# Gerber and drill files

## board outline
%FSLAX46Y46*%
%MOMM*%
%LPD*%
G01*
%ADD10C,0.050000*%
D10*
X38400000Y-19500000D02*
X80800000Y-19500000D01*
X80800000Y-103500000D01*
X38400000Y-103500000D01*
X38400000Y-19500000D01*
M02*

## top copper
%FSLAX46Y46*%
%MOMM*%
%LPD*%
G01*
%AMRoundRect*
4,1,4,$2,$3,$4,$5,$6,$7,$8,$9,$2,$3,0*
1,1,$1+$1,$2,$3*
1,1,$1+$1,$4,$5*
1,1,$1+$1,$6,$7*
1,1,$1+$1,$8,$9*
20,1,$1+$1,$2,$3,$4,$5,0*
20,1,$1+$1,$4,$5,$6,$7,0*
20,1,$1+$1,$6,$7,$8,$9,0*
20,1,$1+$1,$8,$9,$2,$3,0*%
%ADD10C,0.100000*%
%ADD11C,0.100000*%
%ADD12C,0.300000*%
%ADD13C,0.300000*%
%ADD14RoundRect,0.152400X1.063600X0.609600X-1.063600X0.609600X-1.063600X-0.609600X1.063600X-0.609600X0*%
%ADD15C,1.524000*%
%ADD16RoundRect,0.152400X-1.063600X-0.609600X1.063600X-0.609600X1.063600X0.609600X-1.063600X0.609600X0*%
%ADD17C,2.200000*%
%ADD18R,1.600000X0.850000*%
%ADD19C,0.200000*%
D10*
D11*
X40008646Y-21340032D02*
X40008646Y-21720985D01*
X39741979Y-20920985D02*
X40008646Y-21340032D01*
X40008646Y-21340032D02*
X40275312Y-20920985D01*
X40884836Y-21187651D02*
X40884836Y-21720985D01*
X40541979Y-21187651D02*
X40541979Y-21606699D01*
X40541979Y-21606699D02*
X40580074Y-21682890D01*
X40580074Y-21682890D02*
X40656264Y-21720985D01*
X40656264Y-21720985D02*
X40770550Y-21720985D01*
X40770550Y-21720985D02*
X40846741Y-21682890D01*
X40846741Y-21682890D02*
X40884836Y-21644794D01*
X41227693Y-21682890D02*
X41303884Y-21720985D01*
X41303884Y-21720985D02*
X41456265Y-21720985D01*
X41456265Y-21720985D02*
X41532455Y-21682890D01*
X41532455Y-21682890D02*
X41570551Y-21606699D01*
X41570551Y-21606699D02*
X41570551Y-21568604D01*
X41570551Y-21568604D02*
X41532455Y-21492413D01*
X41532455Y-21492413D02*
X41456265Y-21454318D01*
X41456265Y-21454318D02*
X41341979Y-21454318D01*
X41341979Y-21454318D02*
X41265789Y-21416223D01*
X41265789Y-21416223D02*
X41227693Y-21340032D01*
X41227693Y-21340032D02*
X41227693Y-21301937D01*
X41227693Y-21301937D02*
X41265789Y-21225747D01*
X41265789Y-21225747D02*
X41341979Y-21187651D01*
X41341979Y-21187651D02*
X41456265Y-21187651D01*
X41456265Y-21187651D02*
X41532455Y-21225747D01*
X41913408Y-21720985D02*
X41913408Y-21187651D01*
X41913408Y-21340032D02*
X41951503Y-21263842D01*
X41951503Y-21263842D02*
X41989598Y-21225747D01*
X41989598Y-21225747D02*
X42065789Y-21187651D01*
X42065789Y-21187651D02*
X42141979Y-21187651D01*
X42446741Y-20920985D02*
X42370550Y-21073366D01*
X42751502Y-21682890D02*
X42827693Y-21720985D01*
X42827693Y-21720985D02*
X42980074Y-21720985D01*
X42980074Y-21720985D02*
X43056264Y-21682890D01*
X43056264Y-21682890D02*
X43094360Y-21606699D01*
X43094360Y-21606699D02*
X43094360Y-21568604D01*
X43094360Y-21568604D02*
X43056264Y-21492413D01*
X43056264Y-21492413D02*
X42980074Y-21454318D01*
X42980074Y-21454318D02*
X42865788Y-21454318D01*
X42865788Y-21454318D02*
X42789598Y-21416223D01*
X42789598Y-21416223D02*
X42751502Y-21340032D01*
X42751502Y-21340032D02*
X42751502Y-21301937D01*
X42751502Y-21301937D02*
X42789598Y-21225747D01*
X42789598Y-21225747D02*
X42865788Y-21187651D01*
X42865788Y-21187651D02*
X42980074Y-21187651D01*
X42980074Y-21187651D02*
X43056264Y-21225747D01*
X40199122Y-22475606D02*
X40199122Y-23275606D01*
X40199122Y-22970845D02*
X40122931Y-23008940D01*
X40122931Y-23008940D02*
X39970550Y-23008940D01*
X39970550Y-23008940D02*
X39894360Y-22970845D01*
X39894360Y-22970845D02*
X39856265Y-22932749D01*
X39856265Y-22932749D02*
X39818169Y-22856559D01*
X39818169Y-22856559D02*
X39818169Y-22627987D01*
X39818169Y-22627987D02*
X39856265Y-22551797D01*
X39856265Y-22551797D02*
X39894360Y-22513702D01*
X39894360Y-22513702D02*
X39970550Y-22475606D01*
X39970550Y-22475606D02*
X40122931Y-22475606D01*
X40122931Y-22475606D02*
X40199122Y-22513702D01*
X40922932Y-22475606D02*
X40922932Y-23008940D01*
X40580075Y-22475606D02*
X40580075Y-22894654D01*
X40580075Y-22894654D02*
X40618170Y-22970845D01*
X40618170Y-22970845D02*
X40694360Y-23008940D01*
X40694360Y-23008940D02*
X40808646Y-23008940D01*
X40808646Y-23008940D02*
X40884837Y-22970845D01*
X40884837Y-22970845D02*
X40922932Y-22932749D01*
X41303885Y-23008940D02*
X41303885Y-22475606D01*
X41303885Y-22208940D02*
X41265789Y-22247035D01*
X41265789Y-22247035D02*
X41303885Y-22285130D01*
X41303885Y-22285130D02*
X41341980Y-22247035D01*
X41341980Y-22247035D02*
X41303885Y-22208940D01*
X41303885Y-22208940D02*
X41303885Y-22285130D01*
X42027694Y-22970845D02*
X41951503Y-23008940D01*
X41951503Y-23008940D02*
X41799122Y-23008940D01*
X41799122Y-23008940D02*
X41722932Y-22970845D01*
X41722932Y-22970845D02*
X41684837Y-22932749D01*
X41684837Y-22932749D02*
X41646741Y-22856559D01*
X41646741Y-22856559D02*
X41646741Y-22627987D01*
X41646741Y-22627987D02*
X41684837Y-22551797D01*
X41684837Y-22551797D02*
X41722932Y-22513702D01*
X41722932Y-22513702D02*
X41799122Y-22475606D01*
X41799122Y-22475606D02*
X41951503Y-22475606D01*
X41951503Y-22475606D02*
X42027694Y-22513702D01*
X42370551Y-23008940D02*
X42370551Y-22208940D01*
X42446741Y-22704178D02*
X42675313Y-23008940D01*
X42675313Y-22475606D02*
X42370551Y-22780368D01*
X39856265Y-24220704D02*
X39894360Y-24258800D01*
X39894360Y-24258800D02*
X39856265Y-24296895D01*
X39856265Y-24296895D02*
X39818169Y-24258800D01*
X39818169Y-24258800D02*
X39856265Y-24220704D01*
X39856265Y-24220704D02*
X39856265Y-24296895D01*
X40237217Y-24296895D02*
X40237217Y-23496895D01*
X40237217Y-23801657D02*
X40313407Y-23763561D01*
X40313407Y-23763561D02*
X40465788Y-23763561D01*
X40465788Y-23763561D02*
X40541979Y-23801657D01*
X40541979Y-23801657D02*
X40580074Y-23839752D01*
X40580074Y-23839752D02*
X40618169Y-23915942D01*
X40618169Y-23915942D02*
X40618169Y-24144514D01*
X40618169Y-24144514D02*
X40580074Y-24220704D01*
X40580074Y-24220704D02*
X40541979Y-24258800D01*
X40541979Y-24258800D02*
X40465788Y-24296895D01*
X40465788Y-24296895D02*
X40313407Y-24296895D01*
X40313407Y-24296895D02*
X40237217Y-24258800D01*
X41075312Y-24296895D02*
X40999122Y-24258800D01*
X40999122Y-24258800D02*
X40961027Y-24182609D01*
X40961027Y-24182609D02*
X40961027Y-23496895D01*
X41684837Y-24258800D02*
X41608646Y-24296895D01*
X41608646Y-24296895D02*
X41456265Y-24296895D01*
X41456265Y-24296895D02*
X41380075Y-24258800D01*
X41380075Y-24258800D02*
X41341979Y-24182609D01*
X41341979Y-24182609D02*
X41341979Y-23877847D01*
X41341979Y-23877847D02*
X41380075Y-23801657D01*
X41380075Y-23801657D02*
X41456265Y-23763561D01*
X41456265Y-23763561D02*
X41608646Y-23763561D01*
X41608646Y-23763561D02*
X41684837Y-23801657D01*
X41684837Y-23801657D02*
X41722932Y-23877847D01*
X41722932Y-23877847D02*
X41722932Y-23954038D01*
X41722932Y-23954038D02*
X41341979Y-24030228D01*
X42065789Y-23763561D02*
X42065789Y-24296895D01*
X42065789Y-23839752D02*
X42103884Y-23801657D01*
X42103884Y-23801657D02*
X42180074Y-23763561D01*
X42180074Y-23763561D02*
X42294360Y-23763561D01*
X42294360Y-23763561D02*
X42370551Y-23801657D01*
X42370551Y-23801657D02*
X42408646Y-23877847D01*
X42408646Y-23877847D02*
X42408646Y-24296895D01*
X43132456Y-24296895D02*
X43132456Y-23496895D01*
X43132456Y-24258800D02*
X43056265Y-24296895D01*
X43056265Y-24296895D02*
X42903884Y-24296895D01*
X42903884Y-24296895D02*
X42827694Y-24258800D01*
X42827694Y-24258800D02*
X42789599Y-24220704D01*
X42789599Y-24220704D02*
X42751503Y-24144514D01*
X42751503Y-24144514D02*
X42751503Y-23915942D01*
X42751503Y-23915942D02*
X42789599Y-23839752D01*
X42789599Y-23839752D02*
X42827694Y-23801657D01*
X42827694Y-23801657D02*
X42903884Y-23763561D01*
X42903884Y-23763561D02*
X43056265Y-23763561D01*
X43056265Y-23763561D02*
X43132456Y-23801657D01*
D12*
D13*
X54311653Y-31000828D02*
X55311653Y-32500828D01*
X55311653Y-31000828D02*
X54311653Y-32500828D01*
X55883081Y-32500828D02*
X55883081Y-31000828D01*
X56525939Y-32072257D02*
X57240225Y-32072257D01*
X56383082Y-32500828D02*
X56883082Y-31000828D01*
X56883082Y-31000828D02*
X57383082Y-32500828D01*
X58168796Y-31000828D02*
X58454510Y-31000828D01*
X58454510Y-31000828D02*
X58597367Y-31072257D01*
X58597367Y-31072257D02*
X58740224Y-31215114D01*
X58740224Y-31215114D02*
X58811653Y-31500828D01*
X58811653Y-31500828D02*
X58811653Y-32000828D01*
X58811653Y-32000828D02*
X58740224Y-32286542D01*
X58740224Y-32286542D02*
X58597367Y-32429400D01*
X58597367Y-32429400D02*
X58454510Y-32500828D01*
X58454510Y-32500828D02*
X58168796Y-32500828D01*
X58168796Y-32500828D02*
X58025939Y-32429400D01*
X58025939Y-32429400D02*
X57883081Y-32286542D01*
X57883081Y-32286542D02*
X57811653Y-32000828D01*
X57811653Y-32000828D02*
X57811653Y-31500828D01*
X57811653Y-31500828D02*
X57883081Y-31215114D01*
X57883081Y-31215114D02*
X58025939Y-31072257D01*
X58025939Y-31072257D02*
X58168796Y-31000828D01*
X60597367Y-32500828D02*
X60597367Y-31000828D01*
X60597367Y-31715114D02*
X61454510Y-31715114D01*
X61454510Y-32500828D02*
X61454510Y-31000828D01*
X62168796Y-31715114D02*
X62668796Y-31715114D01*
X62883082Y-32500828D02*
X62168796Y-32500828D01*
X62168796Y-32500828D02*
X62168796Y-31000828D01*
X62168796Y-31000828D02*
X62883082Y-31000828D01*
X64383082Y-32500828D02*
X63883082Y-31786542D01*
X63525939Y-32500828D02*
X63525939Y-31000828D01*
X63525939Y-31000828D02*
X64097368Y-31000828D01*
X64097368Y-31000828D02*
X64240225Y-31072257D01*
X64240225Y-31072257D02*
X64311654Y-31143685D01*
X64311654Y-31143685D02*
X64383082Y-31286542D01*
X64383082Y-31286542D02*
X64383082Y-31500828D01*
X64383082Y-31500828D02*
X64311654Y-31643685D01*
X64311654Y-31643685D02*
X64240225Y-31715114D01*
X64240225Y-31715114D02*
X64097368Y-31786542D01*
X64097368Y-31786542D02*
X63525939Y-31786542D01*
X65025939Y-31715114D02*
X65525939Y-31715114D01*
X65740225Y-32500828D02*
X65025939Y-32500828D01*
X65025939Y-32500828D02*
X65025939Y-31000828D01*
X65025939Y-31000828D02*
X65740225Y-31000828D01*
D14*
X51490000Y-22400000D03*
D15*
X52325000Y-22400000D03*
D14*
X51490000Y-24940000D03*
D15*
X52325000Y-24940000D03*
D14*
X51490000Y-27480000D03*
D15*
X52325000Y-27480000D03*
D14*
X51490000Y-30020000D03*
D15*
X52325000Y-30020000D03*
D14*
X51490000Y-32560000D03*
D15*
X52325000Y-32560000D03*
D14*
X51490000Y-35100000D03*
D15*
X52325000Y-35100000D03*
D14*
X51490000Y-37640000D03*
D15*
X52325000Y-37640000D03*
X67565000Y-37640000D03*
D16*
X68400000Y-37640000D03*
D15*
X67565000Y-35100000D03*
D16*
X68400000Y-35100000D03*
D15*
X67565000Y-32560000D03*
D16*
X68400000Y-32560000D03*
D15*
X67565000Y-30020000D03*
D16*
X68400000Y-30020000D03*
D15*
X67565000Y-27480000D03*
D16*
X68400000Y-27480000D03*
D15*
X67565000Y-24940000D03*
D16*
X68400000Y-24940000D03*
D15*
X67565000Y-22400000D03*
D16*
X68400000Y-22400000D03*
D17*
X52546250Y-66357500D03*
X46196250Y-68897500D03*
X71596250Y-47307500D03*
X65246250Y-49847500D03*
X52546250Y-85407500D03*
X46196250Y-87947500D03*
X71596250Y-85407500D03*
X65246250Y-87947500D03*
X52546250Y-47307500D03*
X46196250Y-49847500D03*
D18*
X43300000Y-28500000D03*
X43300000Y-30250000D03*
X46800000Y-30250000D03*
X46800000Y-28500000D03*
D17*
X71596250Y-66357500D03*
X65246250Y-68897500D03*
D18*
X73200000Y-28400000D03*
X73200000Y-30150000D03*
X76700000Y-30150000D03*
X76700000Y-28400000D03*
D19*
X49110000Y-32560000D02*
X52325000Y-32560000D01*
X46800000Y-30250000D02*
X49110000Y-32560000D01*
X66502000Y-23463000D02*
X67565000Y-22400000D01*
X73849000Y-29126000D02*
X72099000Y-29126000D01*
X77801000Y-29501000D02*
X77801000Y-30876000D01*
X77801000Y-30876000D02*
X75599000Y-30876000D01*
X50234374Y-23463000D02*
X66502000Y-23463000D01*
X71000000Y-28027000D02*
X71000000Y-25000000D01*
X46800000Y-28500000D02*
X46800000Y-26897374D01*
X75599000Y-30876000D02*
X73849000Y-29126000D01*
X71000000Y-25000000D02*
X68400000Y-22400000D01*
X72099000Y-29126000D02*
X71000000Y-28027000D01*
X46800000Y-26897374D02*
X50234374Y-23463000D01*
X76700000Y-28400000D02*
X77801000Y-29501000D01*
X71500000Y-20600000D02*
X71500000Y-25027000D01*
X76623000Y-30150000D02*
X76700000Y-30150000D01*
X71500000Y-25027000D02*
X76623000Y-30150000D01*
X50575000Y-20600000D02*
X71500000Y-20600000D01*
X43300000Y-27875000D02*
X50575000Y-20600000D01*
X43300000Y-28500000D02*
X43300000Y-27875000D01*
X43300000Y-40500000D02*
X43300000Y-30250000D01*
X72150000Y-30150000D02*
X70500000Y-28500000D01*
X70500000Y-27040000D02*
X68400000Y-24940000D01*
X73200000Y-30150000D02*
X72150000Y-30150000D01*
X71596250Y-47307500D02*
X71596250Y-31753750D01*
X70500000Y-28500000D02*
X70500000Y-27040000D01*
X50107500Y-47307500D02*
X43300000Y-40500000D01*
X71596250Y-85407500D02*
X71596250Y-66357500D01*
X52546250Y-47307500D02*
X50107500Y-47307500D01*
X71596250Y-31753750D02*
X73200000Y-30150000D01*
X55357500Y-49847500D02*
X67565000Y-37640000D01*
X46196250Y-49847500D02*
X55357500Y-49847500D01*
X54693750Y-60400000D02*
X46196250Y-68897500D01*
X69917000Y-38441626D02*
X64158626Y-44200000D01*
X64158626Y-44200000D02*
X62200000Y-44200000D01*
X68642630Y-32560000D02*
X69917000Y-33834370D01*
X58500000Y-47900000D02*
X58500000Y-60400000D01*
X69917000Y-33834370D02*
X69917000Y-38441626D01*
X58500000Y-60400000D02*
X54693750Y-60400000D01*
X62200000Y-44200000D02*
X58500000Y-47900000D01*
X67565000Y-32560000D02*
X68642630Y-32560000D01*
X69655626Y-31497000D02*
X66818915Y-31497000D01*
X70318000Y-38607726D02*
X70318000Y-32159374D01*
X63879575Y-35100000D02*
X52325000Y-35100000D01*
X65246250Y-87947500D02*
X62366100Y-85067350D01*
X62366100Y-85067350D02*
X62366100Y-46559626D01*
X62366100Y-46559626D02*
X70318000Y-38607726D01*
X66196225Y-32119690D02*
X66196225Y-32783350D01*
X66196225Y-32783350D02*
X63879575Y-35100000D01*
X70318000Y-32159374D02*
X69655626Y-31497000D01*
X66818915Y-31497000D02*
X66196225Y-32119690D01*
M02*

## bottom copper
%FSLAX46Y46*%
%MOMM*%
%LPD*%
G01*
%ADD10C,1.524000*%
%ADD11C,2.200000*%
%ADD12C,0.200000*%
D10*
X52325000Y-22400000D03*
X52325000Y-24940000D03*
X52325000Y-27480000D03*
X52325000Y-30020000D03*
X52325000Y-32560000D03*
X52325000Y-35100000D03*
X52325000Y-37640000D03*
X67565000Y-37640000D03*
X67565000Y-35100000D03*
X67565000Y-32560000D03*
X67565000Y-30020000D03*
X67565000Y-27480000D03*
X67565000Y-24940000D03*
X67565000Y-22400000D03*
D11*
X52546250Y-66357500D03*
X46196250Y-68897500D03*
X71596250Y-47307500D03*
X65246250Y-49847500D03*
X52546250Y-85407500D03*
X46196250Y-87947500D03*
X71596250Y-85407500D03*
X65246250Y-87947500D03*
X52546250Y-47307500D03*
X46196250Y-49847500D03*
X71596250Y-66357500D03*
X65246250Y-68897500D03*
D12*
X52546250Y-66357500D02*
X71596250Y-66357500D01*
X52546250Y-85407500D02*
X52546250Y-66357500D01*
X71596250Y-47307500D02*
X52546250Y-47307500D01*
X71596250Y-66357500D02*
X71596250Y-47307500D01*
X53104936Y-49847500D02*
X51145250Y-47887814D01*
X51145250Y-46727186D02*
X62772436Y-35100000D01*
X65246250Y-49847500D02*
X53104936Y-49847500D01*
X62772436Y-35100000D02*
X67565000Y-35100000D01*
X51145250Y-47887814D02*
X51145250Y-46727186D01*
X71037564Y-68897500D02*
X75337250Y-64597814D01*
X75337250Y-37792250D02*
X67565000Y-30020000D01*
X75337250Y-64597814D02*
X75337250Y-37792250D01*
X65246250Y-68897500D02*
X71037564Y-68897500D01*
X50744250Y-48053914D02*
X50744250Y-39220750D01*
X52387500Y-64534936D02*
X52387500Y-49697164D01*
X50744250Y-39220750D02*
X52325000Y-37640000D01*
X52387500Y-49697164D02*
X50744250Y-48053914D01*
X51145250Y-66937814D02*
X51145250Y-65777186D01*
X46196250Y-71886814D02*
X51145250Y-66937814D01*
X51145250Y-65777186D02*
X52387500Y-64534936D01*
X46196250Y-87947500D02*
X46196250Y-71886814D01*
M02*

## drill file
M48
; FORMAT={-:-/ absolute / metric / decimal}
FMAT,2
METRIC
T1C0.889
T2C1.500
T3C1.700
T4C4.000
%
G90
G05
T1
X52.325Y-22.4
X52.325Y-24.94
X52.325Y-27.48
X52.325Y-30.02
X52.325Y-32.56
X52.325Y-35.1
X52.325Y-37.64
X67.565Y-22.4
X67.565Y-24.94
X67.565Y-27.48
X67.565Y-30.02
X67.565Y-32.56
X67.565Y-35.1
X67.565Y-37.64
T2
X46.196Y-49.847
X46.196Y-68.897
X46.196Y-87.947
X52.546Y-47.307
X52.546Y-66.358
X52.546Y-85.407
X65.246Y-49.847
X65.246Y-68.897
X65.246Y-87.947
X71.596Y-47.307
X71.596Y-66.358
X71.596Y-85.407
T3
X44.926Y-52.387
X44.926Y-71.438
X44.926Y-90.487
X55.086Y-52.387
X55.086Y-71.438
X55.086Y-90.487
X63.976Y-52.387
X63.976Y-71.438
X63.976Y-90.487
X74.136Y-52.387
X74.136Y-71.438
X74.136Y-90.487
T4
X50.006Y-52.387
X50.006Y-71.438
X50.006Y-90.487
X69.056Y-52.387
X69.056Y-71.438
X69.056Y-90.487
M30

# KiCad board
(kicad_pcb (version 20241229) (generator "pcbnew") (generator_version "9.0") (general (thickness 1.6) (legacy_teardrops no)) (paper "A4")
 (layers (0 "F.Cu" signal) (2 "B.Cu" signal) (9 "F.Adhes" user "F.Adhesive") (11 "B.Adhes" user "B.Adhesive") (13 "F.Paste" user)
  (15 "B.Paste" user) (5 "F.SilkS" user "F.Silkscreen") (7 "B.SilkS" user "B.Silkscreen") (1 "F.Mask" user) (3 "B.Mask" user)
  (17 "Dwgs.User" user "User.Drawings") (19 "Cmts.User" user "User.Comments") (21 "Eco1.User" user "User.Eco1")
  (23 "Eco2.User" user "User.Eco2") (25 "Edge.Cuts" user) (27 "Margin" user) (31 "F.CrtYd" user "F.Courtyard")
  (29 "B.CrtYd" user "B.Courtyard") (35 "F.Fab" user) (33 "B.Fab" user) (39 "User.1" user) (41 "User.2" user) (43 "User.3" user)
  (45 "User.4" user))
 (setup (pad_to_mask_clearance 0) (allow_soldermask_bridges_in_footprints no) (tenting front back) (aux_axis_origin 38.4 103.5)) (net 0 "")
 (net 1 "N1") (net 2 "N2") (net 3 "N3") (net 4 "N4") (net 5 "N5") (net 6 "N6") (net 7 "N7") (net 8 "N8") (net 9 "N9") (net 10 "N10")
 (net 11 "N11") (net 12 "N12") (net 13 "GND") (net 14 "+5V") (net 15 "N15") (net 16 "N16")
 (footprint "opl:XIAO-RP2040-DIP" (layer "F.Cu") (at 59.945 30.02)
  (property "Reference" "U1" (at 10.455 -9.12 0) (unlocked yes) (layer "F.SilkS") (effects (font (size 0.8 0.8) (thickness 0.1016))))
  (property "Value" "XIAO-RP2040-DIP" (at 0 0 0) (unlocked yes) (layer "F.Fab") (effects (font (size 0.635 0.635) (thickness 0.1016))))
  (pad "1" smd roundrect (at -8.455 -7.62 180) (size 2.432 1.524) (layers "F.Cu" "F.Mask") (roundrect_rratio 0.1) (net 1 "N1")
   (thermal_bridge_angle 45))
  (pad "1" thru_hole circle (at -7.62 -7.62 180) (size 1.524 1.524) (drill 0.889) (layers "*.Cu" "*.Mask") (remove_unused_layers no)
   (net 1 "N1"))
  (pad "2" smd roundrect (at -8.455 -5.08 180) (size 2.432 1.524) (layers "F.Cu" "F.Mask") (roundrect_rratio 0.1) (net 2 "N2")
   (thermal_bridge_angle 45))
  (pad "2" thru_hole circle (at -7.62 -5.08 180) (size 1.524 1.524) (drill 0.889) (layers "*.Cu" "*.Mask") (remove_unused_layers no)
   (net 2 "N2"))
  (pad "3" smd roundrect (at -8.455 -2.54 180) (size 2.432 1.524) (layers "F.Cu" "F.Mask") (roundrect_rratio 0.1) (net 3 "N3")
   (thermal_bridge_angle 45))
  (pad "3" thru_hole circle (at -7.62 -2.54 180) (size 1.524 1.524) (drill 0.889) (layers "*.Cu" "*.Mask") (remove_unused_layers no)
   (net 3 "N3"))
  (pad "4" smd roundrect (at -8.455 0 180) (size 2.432 1.524) (layers "F.Cu" "F.Mask") (roundrect_rratio 0.1) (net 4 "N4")
   (thermal_bridge_angle 45))
  (pad "4" thru_hole circle (at -7.62 0 180) (size 1.524 1.524) (drill 0.889) (layers "*.Cu" "*.Mask") (remove_unused_layers no)
   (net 4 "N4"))
  (pad "5" smd roundrect (at -8.455 2.54 180) (size 2.432 1.524) (layers "F.Cu" "F.Mask") (roundrect_rratio 0.1) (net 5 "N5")
   (thermal_bridge_angle 45))
  (pad "5" thru_hole circle (at -7.62 2.54 180) (size 1.524 1.524) (drill 0.889) (layers "*.Cu" "*.Mask") (remove_unused_layers no)
   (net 5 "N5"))
  (pad "6" smd roundrect (at -8.455 5.08 180) (size 2.432 1.524) (layers "F.Cu" "F.Mask") (roundrect_rratio 0.1) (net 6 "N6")
   (thermal_bridge_angle 45))
  (pad "6" thru_hole circle (at -7.62 5.08 180) (size 1.524 1.524) (drill 0.889) (layers "*.Cu" "*.Mask") (remove_unused_layers no)
   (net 6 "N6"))
  (pad "7" smd roundrect (at -8.455 7.62 180) (size 2.432 1.524) (layers "F.Cu" "F.Mask") (roundrect_rratio 0.1) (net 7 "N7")
   (thermal_bridge_angle 45))
  (pad "7" thru_hole circle (at -7.62 7.62 180) (size 1.524 1.524) (drill 0.889) (layers "*.Cu" "*.Mask") (remove_unused_layers no)
   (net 7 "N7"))
  (pad "8" thru_hole circle (at 7.62 7.62) (size 1.524 1.524) (drill 0.889) (layers "*.Cu" "*.Mask") (remove_unused_layers no) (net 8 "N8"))
  (pad "8" smd roundrect (at 8.455 7.62) (size 2.432 1.524) (layers "F.Cu" "F.Mask") (roundrect_rratio 0.1) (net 8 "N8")
   (thermal_bridge_angle 45))
  (pad "9" thru_hole circle (at 7.62 5.08) (size 1.524 1.524) (drill 0.889) (layers "*.Cu" "*.Mask") (remove_unused_layers no) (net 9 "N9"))
  (pad "9" smd roundrect (at 8.455 5.08) (size 2.432 1.524) (layers "F.Cu" "F.Mask") (roundrect_rratio 0.1) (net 9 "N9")
   (thermal_bridge_angle 45))
  (pad "10" thru_hole circle (at 7.62 2.54) (size 1.524 1.524) (drill 0.889) (layers "*.Cu" "*.Mask") (remove_unused_layers no)
   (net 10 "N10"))
  (pad "10" smd roundrect (at 8.455 2.54) (size 2.432 1.524) (layers "F.Cu" "F.Mask") (roundrect_rratio 0.1) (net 10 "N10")
   (thermal_bridge_angle 45))
  (pad "11" thru_hole circle (at 7.62 0) (size 1.524 1.524) (drill 0.889) (layers "*.Cu" "*.Mask") (remove_unused_layers no) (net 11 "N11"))
  (pad "11" smd roundrect (at 8.455 0) (size 2.432 1.524) (layers "F.Cu" "F.Mask") (roundrect_rratio 0.1) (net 11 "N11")
   (thermal_bridge_angle 45))
  (pad "12" thru_hole circle (at 7.62 -2.54) (size 1.524 1.524) (drill 0.889) (layers "*.Cu" "*.Mask") (remove_unused_layers no)
   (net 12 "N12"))
  (pad "12" smd roundrect (at 8.455 -2.54) (size 2.432 1.524) (layers "F.Cu" "F.Mask") (roundrect_rratio 0.1) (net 12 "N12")
   (thermal_bridge_angle 45))
  (pad "13" thru_hole circle (at 7.62 -5.08) (size 1.524 1.524) (drill 0.889) (layers "*.Cu" "*.Mask") (remove_unused_layers no)
   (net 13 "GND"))
  (pad "13" smd roundrect (at 8.455 -5.08) (size 2.432 1.524) (layers "F.Cu" "F.Mask") (roundrect_rratio 0.1) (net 13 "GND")
   (thermal_bridge_angle 45))
  (pad "14" thru_hole circle (at 7.62 -7.62) (size 1.524 1.524) (drill 0.889) (layers "*.Cu" "*.Mask") (remove_unused_layers no)
   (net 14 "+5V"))
  (pad "14" smd roundrect (at 8.455 -7.62) (size 2.432 1.524) (layers "F.Cu" "F.Mask") (roundrect_rratio 0.1) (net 14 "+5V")
   (thermal_bridge_angle 45)))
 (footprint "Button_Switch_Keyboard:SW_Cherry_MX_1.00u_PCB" (layer "F.Cu") (at 52.54625 66.3575)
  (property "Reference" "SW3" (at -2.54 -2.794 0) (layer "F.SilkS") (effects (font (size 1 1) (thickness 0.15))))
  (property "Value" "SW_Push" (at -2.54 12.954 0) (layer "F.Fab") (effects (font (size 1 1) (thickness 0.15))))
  (pad "" np_thru_hole circle (at -7.62 5.08) (size 1.7 1.7) (drill 1.7) (layers "*.Cu" "*.Mask"))
  (pad "" np_thru_hole circle (at -2.54 5.08) (size 4 4) (drill 4) (layers "*.Cu" "*.Mask"))
  (pad "" np_thru_hole circle (at 2.54 5.08) (size 1.7 1.7) (drill 1.7) (layers "*.Cu" "*.Mask"))
  (pad "1" thru_hole circle (at 0 0) (size 2.2 2.2) (drill 1.5) (layers "*.Cu" "*.Mask") (remove_unused_layers no) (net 13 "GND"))
  (pad "2" thru_hole circle (at -6.35 2.54) (size 2.2 2.2) (drill 1.5) (layers "*.Cu" "*.Mask") (remove_unused_layers no) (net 10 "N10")))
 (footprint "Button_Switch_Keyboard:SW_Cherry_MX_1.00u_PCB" (layer "F.Cu") (at 71.59625 47.3075)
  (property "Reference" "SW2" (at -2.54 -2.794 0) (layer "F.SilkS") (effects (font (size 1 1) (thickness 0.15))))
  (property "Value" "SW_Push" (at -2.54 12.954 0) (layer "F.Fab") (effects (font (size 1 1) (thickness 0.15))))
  (pad "" np_thru_hole circle (at -7.62 5.08) (size 1.7 1.7) (drill 1.7) (layers "*.Cu" "*.Mask"))
  (pad "" np_thru_hole circle (at -2.54 5.08) (size 4 4) (drill 4) (layers "*.Cu" "*.Mask"))
  (pad "" np_thru_hole circle (at 2.54 5.08) (size 1.7 1.7) (drill 1.7) (layers "*.Cu" "*.Mask"))
  (pad "1" thru_hole circle (at 0 0) (size 2.2 2.2) (drill 1.5) (layers "*.Cu" "*.Mask") (remove_unused_layers no) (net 13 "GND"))
  (pad "2" thru_hole circle (at -6.35 2.54) (size 2.2 2.2) (drill 1.5) (layers "*.Cu" "*.Mask") (remove_unused_layers no) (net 9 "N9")))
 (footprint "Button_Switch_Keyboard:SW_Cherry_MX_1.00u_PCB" (layer "F.Cu") (at 52.54625 85.4075)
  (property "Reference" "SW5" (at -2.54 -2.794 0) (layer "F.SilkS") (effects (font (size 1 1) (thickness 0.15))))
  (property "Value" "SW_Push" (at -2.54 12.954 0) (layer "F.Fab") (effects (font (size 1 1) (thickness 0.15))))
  (pad "" np_thru_hole circle (at -7.62 5.08) (size 1.7 1.7) (drill 1.7) (layers "*.Cu" "*.Mask"))
  (pad "" np_thru_hole circle (at -2.54 5.08) (size 4 4) (drill 4) (layers "*.Cu" "*.Mask"))
  (pad "" np_thru_hole circle (at 2.54 5.08) (size 1.7 1.7) (drill 1.7) (layers "*.Cu" "*.Mask"))
  (pad "1" thru_hole circle (at 0 0) (size 2.2 2.2) (drill 1.5) (layers "*.Cu" "*.Mask") (remove_unused_layers no) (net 13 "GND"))
  (pad "2" thru_hole circle (at -6.35 2.54) (size 2.2 2.2) (drill 1.5) (layers "*.Cu" "*.Mask") (remove_unused_layers no) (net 7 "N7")))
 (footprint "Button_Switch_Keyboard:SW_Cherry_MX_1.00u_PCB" (layer "F.Cu") (at 71.59625 85.4075)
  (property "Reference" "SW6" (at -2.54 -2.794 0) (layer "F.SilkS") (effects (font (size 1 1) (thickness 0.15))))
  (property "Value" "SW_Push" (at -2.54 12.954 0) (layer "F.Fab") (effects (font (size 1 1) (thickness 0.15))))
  (pad "" np_thru_hole circle (at -7.62 5.08) (size 1.7 1.7) (drill 1.7) (layers "*.Cu" "*.Mask"))
  (pad "" np_thru_hole circle (at -2.54 5.08) (size 4 4) (drill 4) (layers "*.Cu" "*.Mask"))
  (pad "" np_thru_hole circle (at 2.54 5.08) (size 1.7 1.7) (drill 1.7) (layers "*.Cu" "*.Mask"))
  (pad "1" thru_hole circle (at 0 0) (size 2.2 2.2) (drill 1.5) (layers "*.Cu" "*.Mask") (remove_unused_layers no) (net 13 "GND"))
  (pad "2" thru_hole circle (at -6.35 2.54) (size 2.2 2.2) (drill 1.5) (layers "*.Cu" "*.Mask") (remove_unused_layers no) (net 6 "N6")))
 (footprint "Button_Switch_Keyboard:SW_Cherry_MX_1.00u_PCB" (layer "F.Cu") (at 52.54625 47.3075)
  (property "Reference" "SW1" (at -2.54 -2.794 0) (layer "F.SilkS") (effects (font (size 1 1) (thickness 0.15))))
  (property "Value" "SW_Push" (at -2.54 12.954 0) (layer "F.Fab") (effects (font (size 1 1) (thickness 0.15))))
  (pad "" np_thru_hole circle (at -7.62 5.08) (size 1.7 1.7) (drill 1.7) (layers "*.Cu" "*.Mask"))
  (pad "" np_thru_hole circle (at -2.54 5.08) (size 4 4) (drill 4) (layers "*.Cu" "*.Mask"))
  (pad "" np_thru_hole circle (at 2.54 5.08) (size 1.7 1.7) (drill 1.7) (layers "*.Cu" "*.Mask"))
  (pad "1" thru_hole circle (at 0 0) (size 2.2 2.2) (drill 1.5) (layers "*.Cu" "*.Mask") (remove_unused_layers no) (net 13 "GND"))
  (pad "2" thru_hole circle (at -6.35 2.54) (size 2.2 2.2) (drill 1.5) (layers "*.Cu" "*.Mask") (remove_unused_layers no) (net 8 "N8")))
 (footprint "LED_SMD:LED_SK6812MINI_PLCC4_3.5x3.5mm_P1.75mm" (layer "F.Cu") (at 45.05 29.375)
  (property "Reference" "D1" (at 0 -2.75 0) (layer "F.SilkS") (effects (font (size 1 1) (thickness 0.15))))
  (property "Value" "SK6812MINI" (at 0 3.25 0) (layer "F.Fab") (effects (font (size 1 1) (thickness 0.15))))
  (pad "1" smd rect (at -1.75 -0.875) (size 1.6 0.85) (layers "F.Cu" "F.Mask" "F.Paste") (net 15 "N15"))
  (pad "2" smd rect (at -1.75 0.875) (size 1.6 0.85) (layers "F.Cu" "F.Mask" "F.Paste") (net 13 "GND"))
  (pad "3" smd rect (at 1.75 0.875) (size 1.6 0.85) (layers "F.Cu" "F.Mask" "F.Paste") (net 5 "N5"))
  (pad "4" smd rect (at 1.75 -0.875) (size 1.6 0.85) (layers "F.Cu" "F.Mask" "F.Paste") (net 14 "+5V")))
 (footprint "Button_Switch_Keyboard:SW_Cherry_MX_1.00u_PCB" (layer "F.Cu") (at 71.59625 66.3575)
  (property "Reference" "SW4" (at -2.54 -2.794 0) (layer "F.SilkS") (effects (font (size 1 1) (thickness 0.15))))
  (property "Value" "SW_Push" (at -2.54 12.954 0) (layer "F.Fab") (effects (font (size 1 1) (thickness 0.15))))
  (pad "" np_thru_hole circle (at -7.62 5.08) (size 1.7 1.7) (drill 1.7) (layers "*.Cu" "*.Mask"))
  (pad "" np_thru_hole circle (at -2.54 5.08) (size 4 4) (drill 4) (layers "*.Cu" "*.Mask"))
  (pad "" np_thru_hole circle (at 2.54 5.08) (size 1.7 1.7) (drill 1.7) (layers "*.Cu" "*.Mask"))
  (pad "1" thru_hole circle (at 0 0) (size 2.2 2.2) (drill 1.5) (layers "*.Cu" "*.Mask") (remove_unused_layers no) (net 13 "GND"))
  (pad "2" thru_hole circle (at -6.35 2.54) (size 2.2 2.2) (drill 1.5) (layers "*.Cu" "*.Mask") (remove_unused_layers no) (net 11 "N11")))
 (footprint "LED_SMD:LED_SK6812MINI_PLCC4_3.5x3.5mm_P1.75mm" (layer "F.Cu") (at 74.95 29.275)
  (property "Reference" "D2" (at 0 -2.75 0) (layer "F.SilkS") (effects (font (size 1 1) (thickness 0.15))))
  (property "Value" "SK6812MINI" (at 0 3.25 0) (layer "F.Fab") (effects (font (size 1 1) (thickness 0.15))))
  (pad "1" smd rect (at -1.75 -0.875) (size 1.6 0.85) (layers "F.Cu" "F.Mask" "F.Paste") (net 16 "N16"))
  (pad "2" smd rect (at -1.75 0.875) (size 1.6 0.85) (layers "F.Cu" "F.Mask" "F.Paste") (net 13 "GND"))
  (pad "3" smd rect (at 1.75 0.875) (size 1.6 0.85) (layers "F.Cu" "F.Mask" "F.Paste") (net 15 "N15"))
  (pad "4" smd rect (at 1.75 -0.875) (size 1.6 0.85) (layers "F.Cu" "F.Mask" "F.Paste") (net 14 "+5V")))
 (gr_rect (start 38.4 19.5) (end 80.8 103.5) (stroke (width 0.05) (type default)) (fill no) (layer "Edge.Cuts"))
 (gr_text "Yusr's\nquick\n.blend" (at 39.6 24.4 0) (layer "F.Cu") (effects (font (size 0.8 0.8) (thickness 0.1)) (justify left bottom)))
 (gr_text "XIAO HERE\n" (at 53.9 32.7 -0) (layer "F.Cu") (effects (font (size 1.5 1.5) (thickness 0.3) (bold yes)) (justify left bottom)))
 (segment (start 49.11 32.56) (end 52.325 32.56) (width 0.2) (layer "F.Cu") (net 5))
 (segment (start 46.8 30.25) (end 49.11 32.56) (width 0.2) (layer "F.Cu") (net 5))
 (segment (start 66.502 23.463) (end 67.565 22.4) (width 0.2) (layer "F.Cu") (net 14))
 (segment (start 73.849 29.126) (end 72.099 29.126) (width 0.2) (layer "F.Cu") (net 14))
 (segment (start 77.801 29.501) (end 77.801 30.876) (width 0.2) (layer "F.Cu") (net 14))
 (segment (start 77.801 30.876) (end 75.599 30.876) (width 0.2) (layer "F.Cu") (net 14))
 (segment (start 50.234374 23.463) (end 66.502 23.463) (width 0.2) (layer "F.Cu") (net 14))
 (segment (start 71 28.027) (end 71 25) (width 0.2) (layer "F.Cu") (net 14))
 (segment (start 46.8 28.5) (end 46.8 26.897374) (width 0.2) (layer "F.Cu") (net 14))
 (segment (start 75.599 30.876) (end 73.849 29.126) (width 0.2) (layer "F.Cu") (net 14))
 (segment (start 71 25) (end 68.4 22.4) (width 0.2) (layer "F.Cu") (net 14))
 (segment (start 72.099 29.126) (end 71 28.027) (width 0.2) (layer "F.Cu") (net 14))
 (segment (start 46.8 26.897374) (end 50.234374 23.463) (width 0.2) (layer "F.Cu") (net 14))
 (segment (start 76.7 28.4) (end 77.801 29.501) (width 0.2) (layer "F.Cu") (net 14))
 (segment (start 71.5 20.6) (end 71.5 25.027) (width 0.2) (layer "F.Cu") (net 15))
 (segment (start 76.623 30.15) (end 76.7 30.15) (width 0.2) (layer "F.Cu") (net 15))
 (segment (start 71.5 25.027) (end 76.623 30.15) (width 0.2) (layer "F.Cu") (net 15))
 (segment (start 50.575 20.6) (end 71.5 20.6) (width 0.2) (layer "F.Cu") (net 15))
 (segment (start 43.3 27.875) (end 50.575 20.6) (width 0.2) (layer "F.Cu") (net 15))
 (segment (start 43.3 28.5) (end 43.3 27.875) (width 0.2) (layer "F.Cu") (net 15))
 (segment (start 43.3 40.5) (end 43.3 30.25) (width 0.2) (layer "F.Cu") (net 13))
 (segment (start 72.15 30.15) (end 70.5 28.5) (width 0.2) (layer "F.Cu") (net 13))
 (segment (start 70.5 27.04) (end 68.4 24.94) (width 0.2) (layer "F.Cu") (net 13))
 (segment (start 73.2 30.15) (end 72.15 30.15) (width 0.2) (layer "F.Cu") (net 13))
 (segment (start 71.59625 47.3075) (end 71.59625 31.75375) (width 0.2) (layer "F.Cu") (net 13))
 (segment (start 70.5 28.5) (end 70.5 27.04) (width 0.2) (layer "F.Cu") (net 13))
 (segment (start 50.1075 47.3075) (end 43.3 40.5) (width 0.2) (layer "F.Cu") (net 13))
 (segment (start 71.59625 85.4075) (end 71.59625 66.3575) (width 0.2) (layer "F.Cu") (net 13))
 (segment (start 52.54625 47.3075) (end 50.1075 47.3075) (width 0.2) (layer "F.Cu") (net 13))
 (segment (start 71.59625 31.75375) (end 73.2 30.15) (width 0.2) (layer "F.Cu") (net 13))
 (segment (start 52.54625 66.3575) (end 71.59625 66.3575) (width 0.2) (layer "B.Cu") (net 13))
 (segment (start 52.54625 85.4075) (end 52.54625 66.3575) (width 0.2) (layer "B.Cu") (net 13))
 (segment (start 71.59625 47.3075) (end 52.54625 47.3075) (width 0.2) (layer "B.Cu") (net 13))
 (segment (start 71.59625 66.3575) (end 71.59625 47.3075) (width 0.2) (layer "B.Cu") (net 13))
 (segment (start 55.3575 49.8475) (end 67.565 37.64) (width 0.2) (layer "F.Cu") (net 8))
 (segment (start 46.19625 49.8475) (end 55.3575 49.8475) (width 0.2) (layer "F.Cu") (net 8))
 (segment (start 53.104936 49.8475) (end 51.14525 47.887814) (width 0.2) (layer "B.Cu") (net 9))
 (segment (start 51.14525 46.727186) (end 62.772436 35.1) (width 0.2) (layer "B.Cu") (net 9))
 (segment (start 65.24625 49.8475) (end 53.104936 49.8475) (width 0.2) (layer "B.Cu") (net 9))
 (segment (start 62.772436 35.1) (end 67.565 35.1) (width 0.2) (layer "B.Cu") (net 9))
 (segment (start 51.14525 47.887814) (end 51.14525 46.727186) (width 0.2) (layer "B.Cu") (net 9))
 (segment (start 54.69375 60.4) (end 46.19625 68.8975) (width 0.2) (layer "F.Cu") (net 10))
 (segment (start 69.917 38.441626) (end 64.158626 44.2) (width 0.2) (layer "F.Cu") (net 10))
 (segment (start 64.158626 44.2) (end 62.2 44.2) (width 0.2) (layer "F.Cu") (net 10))
 (segment (start 68.64263 32.56) (end 69.917 33.83437) (width 0.2) (layer "F.Cu") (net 10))
 (segment (start 58.5 47.9) (end 58.5 60.4) (width 0.2) (layer "F.Cu") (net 10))
 (segment (start 69.917 33.83437) (end 69.917 38.441626) (width 0.2) (layer "F.Cu") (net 10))
 (segment (start 58.5 60.4) (end 54.69375 60.4) (width 0.2) (layer "F.Cu") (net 10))
 (segment (start 62.2 44.2) (end 58.5 47.9) (width 0.2) (layer "F.Cu") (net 10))
 (segment (start 67.565 32.56) (end 68.64263 32.56) (width 0.2) (layer "F.Cu") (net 10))
 (segment (start 71.037564 68.8975) (end 75.33725 64.597814) (width 0.2) (layer "B.Cu") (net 11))
 (segment (start 75.33725 37.79225) (end 67.565 30.02) (width 0.2) (layer "B.Cu") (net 11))
 (segment (start 75.33725 64.597814) (end 75.33725 37.79225) (width 0.2) (layer "B.Cu") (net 11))
 (segment (start 65.24625 68.8975) (end 71.037564 68.8975) (width 0.2) (layer "B.Cu") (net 11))
 (segment (start 50.74425 48.053914) (end 50.74425 39.22075) (width 0.2) (layer "B.Cu") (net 7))
 (segment (start 52.3875 64.534936) (end 52.3875 49.697164) (width 0.2) (layer "B.Cu") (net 7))
 (segment (start 50.74425 39.22075) (end 52.325 37.64) (width 0.2) (layer "B.Cu") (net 7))
 (segment (start 52.3875 49.697164) (end 50.74425 48.053914) (width 0.2) (layer "B.Cu") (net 7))
 (segment (start 51.14525 66.937814) (end 51.14525 65.777186) (width 0.2) (layer "B.Cu") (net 7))
 (segment (start 46.19625 71.886814) (end 51.14525 66.937814) (width 0.2) (layer "B.Cu") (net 7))
 (segment (start 51.14525 65.777186) (end 52.3875 64.534936) (width 0.2) (layer "B.Cu") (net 7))
 (segment (start 46.19625 87.9475) (end 46.19625 71.886814) (width 0.2) (layer "B.Cu") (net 7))
 (segment (start 69.655626 31.497) (end 66.818915 31.497) (width 0.2) (layer "F.Cu") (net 6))
 (segment (start 70.318 38.607726) (end 70.318 32.159374) (width 0.2) (layer "F.Cu") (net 6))
 (segment (start 63.879575 35.1) (end 52.325 35.1) (width 0.2) (layer "F.Cu") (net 6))
 (segment (start 65.24625 87.9475) (end 62.3661 85.06735) (width 0.2) (layer "F.Cu") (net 6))
 (segment (start 62.3661 85.06735) (end 62.3661 46.559626) (width 0.2) (layer "F.Cu") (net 6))
 (segment (start 62.3661 46.559626) (end 70.318 38.607726) (width 0.2) (layer "F.Cu") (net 6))
 (segment (start 66.196225 32.11969) (end 66.196225 32.78335) (width 0.2) (layer "F.Cu") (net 6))
 (segment (start 66.196225 32.78335) (end 63.879575 35.1) (width 0.2) (layer "F.Cu") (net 6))
 (segment (start 70.318 32.159374) (end 69.655626 31.497) (width 0.2) (layer "F.Cu") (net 6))
 (segment (start 66.818915 31.497) (end 66.196225 32.11969) (width 0.2) (layer "F.Cu") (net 6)))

